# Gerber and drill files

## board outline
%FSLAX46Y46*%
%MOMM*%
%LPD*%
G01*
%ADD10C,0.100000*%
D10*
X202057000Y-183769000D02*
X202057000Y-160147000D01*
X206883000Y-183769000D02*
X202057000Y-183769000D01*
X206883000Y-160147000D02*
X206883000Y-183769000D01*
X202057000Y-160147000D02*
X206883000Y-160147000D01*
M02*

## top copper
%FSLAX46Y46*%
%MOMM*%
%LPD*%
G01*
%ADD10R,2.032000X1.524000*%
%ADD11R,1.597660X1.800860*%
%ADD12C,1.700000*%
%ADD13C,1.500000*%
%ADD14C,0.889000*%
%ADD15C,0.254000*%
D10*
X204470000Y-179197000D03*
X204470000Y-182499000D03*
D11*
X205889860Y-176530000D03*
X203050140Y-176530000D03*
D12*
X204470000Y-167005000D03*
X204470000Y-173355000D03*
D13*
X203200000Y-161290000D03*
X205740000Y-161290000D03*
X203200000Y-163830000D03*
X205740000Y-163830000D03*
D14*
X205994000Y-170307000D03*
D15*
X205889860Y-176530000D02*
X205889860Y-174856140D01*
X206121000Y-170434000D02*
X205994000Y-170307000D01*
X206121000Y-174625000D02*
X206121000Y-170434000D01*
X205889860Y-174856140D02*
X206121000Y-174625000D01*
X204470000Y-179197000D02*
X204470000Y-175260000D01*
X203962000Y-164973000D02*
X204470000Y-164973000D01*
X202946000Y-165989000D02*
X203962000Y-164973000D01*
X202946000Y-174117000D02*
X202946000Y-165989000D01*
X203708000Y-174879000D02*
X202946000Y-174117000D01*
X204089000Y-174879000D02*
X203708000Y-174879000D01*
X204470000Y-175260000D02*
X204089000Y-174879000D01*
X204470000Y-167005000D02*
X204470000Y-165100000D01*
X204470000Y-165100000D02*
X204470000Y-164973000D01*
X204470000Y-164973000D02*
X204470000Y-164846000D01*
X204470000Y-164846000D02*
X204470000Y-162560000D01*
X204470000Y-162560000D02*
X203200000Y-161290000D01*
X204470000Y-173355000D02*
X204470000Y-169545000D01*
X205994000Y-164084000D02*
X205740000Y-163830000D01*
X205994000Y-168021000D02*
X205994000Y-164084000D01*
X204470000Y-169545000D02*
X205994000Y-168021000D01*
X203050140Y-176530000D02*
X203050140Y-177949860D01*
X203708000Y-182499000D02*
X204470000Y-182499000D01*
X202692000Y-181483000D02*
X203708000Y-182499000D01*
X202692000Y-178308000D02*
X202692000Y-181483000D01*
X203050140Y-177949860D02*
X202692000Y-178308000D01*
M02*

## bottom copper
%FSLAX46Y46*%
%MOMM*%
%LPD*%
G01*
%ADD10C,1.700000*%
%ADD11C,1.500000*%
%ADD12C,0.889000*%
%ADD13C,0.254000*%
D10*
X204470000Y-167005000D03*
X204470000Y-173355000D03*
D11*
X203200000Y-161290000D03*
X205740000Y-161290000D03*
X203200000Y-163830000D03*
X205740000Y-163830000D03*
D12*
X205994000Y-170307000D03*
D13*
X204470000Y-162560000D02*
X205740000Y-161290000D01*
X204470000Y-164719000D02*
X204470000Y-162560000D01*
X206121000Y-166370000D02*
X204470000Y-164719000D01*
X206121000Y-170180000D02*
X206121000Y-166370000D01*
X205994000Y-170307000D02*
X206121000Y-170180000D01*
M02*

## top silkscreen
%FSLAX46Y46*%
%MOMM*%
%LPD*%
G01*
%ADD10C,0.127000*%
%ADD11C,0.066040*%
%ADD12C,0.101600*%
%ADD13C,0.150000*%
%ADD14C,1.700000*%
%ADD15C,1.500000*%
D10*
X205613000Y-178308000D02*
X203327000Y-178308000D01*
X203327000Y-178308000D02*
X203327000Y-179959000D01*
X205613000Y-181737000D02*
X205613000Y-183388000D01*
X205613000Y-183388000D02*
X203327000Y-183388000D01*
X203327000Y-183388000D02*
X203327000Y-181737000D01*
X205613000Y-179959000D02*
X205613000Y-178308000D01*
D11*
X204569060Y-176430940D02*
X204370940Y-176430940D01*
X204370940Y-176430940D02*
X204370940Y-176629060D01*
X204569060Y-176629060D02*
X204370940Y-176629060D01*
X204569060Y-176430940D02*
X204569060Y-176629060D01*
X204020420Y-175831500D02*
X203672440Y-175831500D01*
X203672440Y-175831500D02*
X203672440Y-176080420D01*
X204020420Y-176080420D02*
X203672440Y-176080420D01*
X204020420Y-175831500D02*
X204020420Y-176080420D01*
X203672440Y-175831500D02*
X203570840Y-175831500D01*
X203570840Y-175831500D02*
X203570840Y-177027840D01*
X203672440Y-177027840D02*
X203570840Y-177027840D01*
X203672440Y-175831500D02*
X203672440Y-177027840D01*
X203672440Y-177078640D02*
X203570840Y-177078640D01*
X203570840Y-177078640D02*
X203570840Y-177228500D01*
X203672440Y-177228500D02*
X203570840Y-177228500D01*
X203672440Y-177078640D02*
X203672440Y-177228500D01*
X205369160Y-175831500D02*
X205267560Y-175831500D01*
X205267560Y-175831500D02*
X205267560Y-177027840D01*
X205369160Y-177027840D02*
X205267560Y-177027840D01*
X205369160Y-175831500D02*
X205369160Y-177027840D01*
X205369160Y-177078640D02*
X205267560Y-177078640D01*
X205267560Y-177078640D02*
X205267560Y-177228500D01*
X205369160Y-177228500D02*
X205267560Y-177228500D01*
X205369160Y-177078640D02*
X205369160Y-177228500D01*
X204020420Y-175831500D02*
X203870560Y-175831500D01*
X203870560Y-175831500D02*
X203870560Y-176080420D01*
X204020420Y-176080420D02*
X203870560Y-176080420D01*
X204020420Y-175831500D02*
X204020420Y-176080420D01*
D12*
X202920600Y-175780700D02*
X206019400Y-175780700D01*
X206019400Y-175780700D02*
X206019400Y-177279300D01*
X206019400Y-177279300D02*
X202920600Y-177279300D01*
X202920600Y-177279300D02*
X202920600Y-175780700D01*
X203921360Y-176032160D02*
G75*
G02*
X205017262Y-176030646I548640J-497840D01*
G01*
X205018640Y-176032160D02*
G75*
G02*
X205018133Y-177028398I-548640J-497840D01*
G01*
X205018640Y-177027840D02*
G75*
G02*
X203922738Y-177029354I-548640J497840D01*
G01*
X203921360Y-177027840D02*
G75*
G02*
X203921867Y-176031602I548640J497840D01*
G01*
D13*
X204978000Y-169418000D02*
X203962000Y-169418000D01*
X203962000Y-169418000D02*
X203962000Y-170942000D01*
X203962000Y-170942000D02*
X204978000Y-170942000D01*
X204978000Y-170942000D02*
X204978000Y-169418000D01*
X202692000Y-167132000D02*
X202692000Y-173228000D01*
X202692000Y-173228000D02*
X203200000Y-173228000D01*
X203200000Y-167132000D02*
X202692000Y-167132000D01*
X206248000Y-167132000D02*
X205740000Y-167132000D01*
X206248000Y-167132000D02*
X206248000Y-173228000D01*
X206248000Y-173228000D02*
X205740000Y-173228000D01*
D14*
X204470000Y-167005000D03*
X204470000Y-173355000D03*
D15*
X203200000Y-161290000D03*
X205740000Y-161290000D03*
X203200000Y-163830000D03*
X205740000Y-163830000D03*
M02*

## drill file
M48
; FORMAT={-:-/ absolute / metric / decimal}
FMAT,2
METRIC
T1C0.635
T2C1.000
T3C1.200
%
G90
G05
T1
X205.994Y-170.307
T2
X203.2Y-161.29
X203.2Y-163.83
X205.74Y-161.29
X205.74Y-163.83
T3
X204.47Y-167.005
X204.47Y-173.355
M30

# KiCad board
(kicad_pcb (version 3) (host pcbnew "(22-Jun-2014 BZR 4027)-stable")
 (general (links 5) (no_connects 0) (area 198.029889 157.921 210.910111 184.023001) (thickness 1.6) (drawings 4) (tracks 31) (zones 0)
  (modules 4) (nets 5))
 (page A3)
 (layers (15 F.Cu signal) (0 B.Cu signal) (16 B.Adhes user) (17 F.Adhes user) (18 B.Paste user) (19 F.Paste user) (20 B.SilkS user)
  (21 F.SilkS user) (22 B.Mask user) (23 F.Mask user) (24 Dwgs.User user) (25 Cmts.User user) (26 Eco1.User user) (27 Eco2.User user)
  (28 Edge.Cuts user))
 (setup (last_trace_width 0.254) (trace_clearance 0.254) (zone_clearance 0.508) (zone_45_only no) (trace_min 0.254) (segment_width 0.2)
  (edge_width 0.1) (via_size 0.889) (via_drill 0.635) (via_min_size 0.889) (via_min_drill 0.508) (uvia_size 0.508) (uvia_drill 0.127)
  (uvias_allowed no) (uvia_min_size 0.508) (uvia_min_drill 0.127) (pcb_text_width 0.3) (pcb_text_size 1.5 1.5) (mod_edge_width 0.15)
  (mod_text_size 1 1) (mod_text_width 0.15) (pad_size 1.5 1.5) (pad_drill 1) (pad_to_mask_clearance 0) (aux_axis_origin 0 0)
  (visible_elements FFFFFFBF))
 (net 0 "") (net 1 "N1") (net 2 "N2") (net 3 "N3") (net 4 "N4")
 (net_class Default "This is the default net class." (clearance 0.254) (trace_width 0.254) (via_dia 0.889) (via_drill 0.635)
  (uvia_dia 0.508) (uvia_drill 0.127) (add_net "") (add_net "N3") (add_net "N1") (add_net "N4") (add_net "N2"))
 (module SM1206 (layer F.Cu) (at 204.47 180.848 270)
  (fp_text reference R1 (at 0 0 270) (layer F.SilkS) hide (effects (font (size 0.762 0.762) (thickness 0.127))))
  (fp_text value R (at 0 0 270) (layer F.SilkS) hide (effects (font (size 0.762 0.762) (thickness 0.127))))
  (fp_line (start -2.54 -1.143) (end -2.54 1.143) (layer F.SilkS) (width 0.127))
  (fp_line (start -2.54 1.143) (end -0.889 1.143) (layer F.SilkS) (width 0.127))
  (fp_line (start 0.889 -1.143) (end 2.54 -1.143) (layer F.SilkS) (width 0.127))
  (fp_line (start 2.54 -1.143) (end 2.54 1.143) (layer F.SilkS) (width 0.127))
  (fp_line (start 2.54 1.143) (end 0.889 1.143) (layer F.SilkS) (width 0.127))
  (fp_line (start -0.889 -1.143) (end -2.54 -1.143) (layer F.SilkS) (width 0.127))
  (pad 1 smd rect (at -1.651 0 270) (size 1.524 2.032) (layers F.Cu F.Paste F.Mask) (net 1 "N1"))
  (pad 2 smd rect (at 1.651 0 270) (size 1.524 2.032) (layers F.Cu F.Paste F.Mask) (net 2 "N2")))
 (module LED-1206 (layer F.Cu) (at 204.47 176.53 180)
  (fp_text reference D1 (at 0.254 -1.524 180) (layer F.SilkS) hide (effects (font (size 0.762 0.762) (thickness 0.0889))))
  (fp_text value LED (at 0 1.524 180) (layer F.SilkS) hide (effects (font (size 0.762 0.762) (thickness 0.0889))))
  (fp_line (start -0.09906 0.09906) (end 0.09906 0.09906) (layer F.SilkS) (width 0.06604))
  (fp_line (start 0.09906 0.09906) (end 0.09906 -0.09906) (layer F.SilkS) (width 0.06604))
  (fp_line (start -0.09906 -0.09906) (end 0.09906 -0.09906) (layer F.SilkS) (width 0.06604))
  (fp_line (start -0.09906 0.09906) (end -0.09906 -0.09906) (layer F.SilkS) (width 0.06604))
  (fp_line (start 0.44958 0.6985) (end 0.79756 0.6985) (layer F.SilkS) (width 0.06604))
  (fp_line (start 0.79756 0.6985) (end 0.79756 0.44958) (layer F.SilkS) (width 0.06604))
  (fp_line (start 0.44958 0.44958) (end 0.79756 0.44958) (layer F.SilkS) (width 0.06604))
  (fp_line (start 0.44958 0.6985) (end 0.44958 0.44958) (layer F.SilkS) (width 0.06604))
  (fp_line (start 0.79756 0.6985) (end 0.89916 0.6985) (layer F.SilkS) (width 0.06604))
  (fp_line (start 0.89916 0.6985) (end 0.89916 -0.49784) (layer F.SilkS) (width 0.06604))
  (fp_line (start 0.79756 -0.49784) (end 0.89916 -0.49784) (layer F.SilkS) (width 0.06604))
  (fp_line (start 0.79756 0.6985) (end 0.79756 -0.49784) (layer F.SilkS) (width 0.06604))
  (fp_line (start 0.79756 -0.54864) (end 0.89916 -0.54864) (layer F.SilkS) (width 0.06604))
  (fp_line (start 0.89916 -0.54864) (end 0.89916 -0.6985) (layer F.SilkS) (width 0.06604))
  (fp_line (start 0.79756 -0.6985) (end 0.89916 -0.6985) (layer F.SilkS) (width 0.06604))
  (fp_line (start 0.79756 -0.54864) (end 0.79756 -0.6985) (layer F.SilkS) (width 0.06604))
  (fp_line (start -0.89916 0.6985) (end -0.79756 0.6985) (layer F.SilkS) (width 0.06604))
  (fp_line (start -0.79756 0.6985) (end -0.79756 -0.49784) (layer F.SilkS) (width 0.06604))
  (fp_line (start -0.89916 -0.49784) (end -0.79756 -0.49784) (layer F.SilkS) (width 0.06604))
  (fp_line (start -0.89916 0.6985) (end -0.89916 -0.49784) (layer F.SilkS) (width 0.06604))
  (fp_line (start -0.89916 -0.54864) (end -0.79756 -0.54864) (layer F.SilkS) (width 0.06604))
  (fp_line (start -0.79756 -0.54864) (end -0.79756 -0.6985) (layer F.SilkS) (width 0.06604))
  (fp_line (start -0.89916 -0.6985) (end -0.79756 -0.6985) (layer F.SilkS) (width 0.06604))
  (fp_line (start -0.89916 -0.54864) (end -0.89916 -0.6985) (layer F.SilkS) (width 0.06604))
  (fp_line (start 0.44958 0.6985) (end 0.59944 0.6985) (layer F.SilkS) (width 0.06604))
  (fp_line (start 0.59944 0.6985) (end 0.59944 0.44958) (layer F.SilkS) (width 0.06604))
  (fp_line (start 0.44958 0.44958) (end 0.59944 0.44958) (layer F.SilkS) (width 0.06604))
  (fp_line (start 0.44958 0.6985) (end 0.44958 0.44958) (layer F.SilkS) (width 0.06604))
  (fp_line (start 1.5494 0.7493) (end -1.5494 0.7493) (layer F.SilkS) (width 0.1016))
  (fp_line (start -1.5494 0.7493) (end -1.5494 -0.7493) (layer F.SilkS) (width 0.1016))
  (fp_line (start -1.5494 -0.7493) (end 1.5494 -0.7493) (layer F.SilkS) (width 0.1016))
  (fp_line (start 1.5494 -0.7493) (end 1.5494 0.7493) (layer F.SilkS) (width 0.1016))
  (fp_arc (start 0 0) (end 0.54864 0.49784) (angle 95.4) (layer F.SilkS) (width 0.1016))
  (fp_arc (start 0 0) (end -0.54864 0.49784) (angle 84.5) (layer F.SilkS) (width 0.1016))
  (fp_arc (start 0 0) (end -0.54864 -0.49784) (angle 95.4) (layer F.SilkS) (width 0.1016))
  (fp_arc (start 0 0) (end 0.54864 -0.49784) (angle 84.5) (layer F.SilkS) (width 0.1016))
  (pad 1 smd rect (at -1.41986 0 180) (size 1.59766 1.80086) (layers F.Cu F.Paste F.Mask) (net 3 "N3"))
  (pad 2 smd rect (at 1.41986 0 180) (size 1.59766 1.80086) (layers F.Cu F.Paste F.Mask) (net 2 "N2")))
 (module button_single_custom (layer F.Cu) (at 204.47 170.18 270)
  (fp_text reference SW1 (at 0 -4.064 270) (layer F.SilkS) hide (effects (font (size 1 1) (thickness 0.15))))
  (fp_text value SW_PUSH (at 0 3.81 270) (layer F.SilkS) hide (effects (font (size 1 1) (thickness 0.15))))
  (fp_line (start -0.762 -0.508) (end -0.762 0.508) (layer F.SilkS) (width 0.15))
  (fp_line (start -0.762 0.508) (end 0.762 0.508) (layer F.SilkS) (width 0.15))
  (fp_line (start 0.762 0.508) (end 0.762 -0.508) (layer F.SilkS) (width 0.15))
  (fp_line (start 0.762 -0.508) (end -0.762 -0.508) (layer F.SilkS) (width 0.15))
  (fp_line (start -3.048 1.778) (end 3.048 1.778) (layer F.SilkS) (width 0.15))
  (fp_line (start 3.048 1.778) (end 3.048 1.27) (layer F.SilkS) (width 0.15))
  (fp_line (start -3.048 1.27) (end -3.048 1.778) (layer F.SilkS) (width 0.15))
  (fp_line (start -3.048 -1.778) (end -3.048 -1.27) (layer F.SilkS) (width 0.15))
  (fp_line (start -3.048 -1.778) (end 3.048 -1.778) (layer F.SilkS) (width 0.15))
  (fp_line (start 3.048 -1.778) (end 3.048 -1.27) (layer F.SilkS) (width 0.15))
  (pad 1 thru_hole circle (at -3.175 0 270) (size 1.7 1.7) (drill 1.2) (layers *.Cu *.Mask F.SilkS) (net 1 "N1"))
  (pad 2 thru_hole circle (at 3.175 0 270) (size 1.7 1.7) (drill 1.2) (layers *.Cu *.Mask F.SilkS) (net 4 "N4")))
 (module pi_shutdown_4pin (layer F.Cu) (at 204.47 162.56)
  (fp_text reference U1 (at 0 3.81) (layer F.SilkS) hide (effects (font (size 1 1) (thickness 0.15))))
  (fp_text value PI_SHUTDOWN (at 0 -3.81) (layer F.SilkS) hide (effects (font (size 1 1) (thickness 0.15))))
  (pad 14 thru_hole circle (at -1.27 -1.27) (size 1.5 1.5) (drill 1) (layers *.Cu *.Mask F.SilkS) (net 1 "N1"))
  (pad 16 thru_hole circle (at 1.27 -1.27) (size 1.5 1.5) (drill 1) (layers *.Cu *.Mask F.SilkS) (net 3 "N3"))
  (pad 13 thru_hole circle (at -1.27 1.27) (size 1.5 1.5) (drill 1) (layers *.Cu *.Mask F.SilkS))
  (pad 15 thru_hole circle (at 1.27 1.27) (size 1.5 1.5) (drill 1) (layers *.Cu *.Mask F.SilkS) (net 4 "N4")))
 (gr_line (start 202.057 183.769) (end 202.057 160.147) (angle 90) (layer Edge.Cuts) (width 0.1))
 (gr_line (start 206.883 183.769) (end 202.057 183.769) (angle 90) (layer Edge.Cuts) (width 0.1))
 (gr_line (start 206.883 160.147) (end 206.883 183.769) (angle 90) (layer Edge.Cuts) (width 0.1))
 (gr_line (start 202.057 160.147) (end 206.883 160.147) (angle 90) (layer Edge.Cuts) (width 0.1))
 (segment (start 205.88986 176.53) (end 205.88986 174.85614) (width 0.254) (layer F.Cu) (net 3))
 (segment (start 204.47 162.56) (end 205.74 161.29) (width 0.254) (layer B.Cu) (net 3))
 (segment (start 204.47 164.719) (end 204.47 162.56) (width 0.254) (layer B.Cu) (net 3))
 (segment (start 206.121 166.37) (end 204.47 164.719) (width 0.254) (layer B.Cu) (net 3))
 (segment (start 206.121 170.18) (end 206.121 166.37) (width 0.254) (layer B.Cu) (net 3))
 (segment (start 205.994 170.307) (end 206.121 170.18) (width 0.254) (layer B.Cu) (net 3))
 (via (at 205.994 170.307) (size 0.889) (layers F.Cu B.Cu) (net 3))
 (segment (start 206.121 170.434) (end 205.994 170.307) (width 0.254) (layer F.Cu) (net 3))
 (segment (start 206.121 174.625) (end 206.121 170.434) (width 0.254) (layer F.Cu) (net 3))
 (segment (start 205.88986 174.85614) (end 206.121 174.625) (width 0.254) (layer F.Cu) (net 3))
 (segment (start 204.47 179.197) (end 204.47 175.26) (width 0.254) (layer F.Cu) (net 1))
 (segment (start 203.962 164.973) (end 204.47 164.973) (width 0.254) (layer F.Cu) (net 1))
 (segment (start 202.946 165.989) (end 203.962 164.973) (width 0.254) (layer F.Cu) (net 1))
 (segment (start 202.946 174.117) (end 202.946 165.989) (width 0.254) (layer F.Cu) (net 1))
 (segment (start 203.708 174.879) (end 202.946 174.117) (width 0.254) (layer F.Cu) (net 1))
 (segment (start 204.089 174.879) (end 203.708 174.879) (width 0.254) (layer F.Cu) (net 1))
 (segment (start 204.47 175.26) (end 204.089 174.879) (width 0.254) (layer F.Cu) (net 1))
 (segment (start 204.47 167.005) (end 204.47 165.1) (width 0.254) (layer F.Cu) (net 1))
 (segment (start 204.47 165.1) (end 204.47 164.973) (width 0.254) (layer F.Cu) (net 1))
 (segment (start 204.47 164.973) (end 204.47 164.846) (width 0.254) (layer F.Cu) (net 1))
 (segment (start 204.47 164.846) (end 204.47 162.56) (width 0.254) (layer F.Cu) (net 1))
 (segment (start 204.47 162.56) (end 203.2 161.29) (width 0.254) (layer F.Cu) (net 1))
 (segment (start 204.47 173.355) (end 204.47 169.545) (width 0.254) (layer F.Cu) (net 4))
 (segment (start 205.994 164.084) (end 205.74 163.83) (width 0.254) (layer F.Cu) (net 4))
 (segment (start 205.994 168.021) (end 205.994 164.084) (width 0.254) (layer F.Cu) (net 4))
 (segment (start 204.47 169.545) (end 205.994 168.021) (width 0.254) (layer F.Cu) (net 4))
 (segment (start 203.05014 176.53) (end 203.05014 177.94986) (width 0.254) (layer F.Cu) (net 2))
 (segment (start 203.708 182.499) (end 204.47 182.499) (width 0.254) (layer F.Cu) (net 2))
 (segment (start 202.692 181.483) (end 203.708 182.499) (width 0.254) (layer F.Cu) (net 2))
 (segment (start 202.692 178.308) (end 202.692 181.483) (width 0.254) (layer F.Cu) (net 2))
 (segment (start 203.05014 177.94986) (end 202.692 178.308) (width 0.254) (layer F.Cu) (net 2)))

